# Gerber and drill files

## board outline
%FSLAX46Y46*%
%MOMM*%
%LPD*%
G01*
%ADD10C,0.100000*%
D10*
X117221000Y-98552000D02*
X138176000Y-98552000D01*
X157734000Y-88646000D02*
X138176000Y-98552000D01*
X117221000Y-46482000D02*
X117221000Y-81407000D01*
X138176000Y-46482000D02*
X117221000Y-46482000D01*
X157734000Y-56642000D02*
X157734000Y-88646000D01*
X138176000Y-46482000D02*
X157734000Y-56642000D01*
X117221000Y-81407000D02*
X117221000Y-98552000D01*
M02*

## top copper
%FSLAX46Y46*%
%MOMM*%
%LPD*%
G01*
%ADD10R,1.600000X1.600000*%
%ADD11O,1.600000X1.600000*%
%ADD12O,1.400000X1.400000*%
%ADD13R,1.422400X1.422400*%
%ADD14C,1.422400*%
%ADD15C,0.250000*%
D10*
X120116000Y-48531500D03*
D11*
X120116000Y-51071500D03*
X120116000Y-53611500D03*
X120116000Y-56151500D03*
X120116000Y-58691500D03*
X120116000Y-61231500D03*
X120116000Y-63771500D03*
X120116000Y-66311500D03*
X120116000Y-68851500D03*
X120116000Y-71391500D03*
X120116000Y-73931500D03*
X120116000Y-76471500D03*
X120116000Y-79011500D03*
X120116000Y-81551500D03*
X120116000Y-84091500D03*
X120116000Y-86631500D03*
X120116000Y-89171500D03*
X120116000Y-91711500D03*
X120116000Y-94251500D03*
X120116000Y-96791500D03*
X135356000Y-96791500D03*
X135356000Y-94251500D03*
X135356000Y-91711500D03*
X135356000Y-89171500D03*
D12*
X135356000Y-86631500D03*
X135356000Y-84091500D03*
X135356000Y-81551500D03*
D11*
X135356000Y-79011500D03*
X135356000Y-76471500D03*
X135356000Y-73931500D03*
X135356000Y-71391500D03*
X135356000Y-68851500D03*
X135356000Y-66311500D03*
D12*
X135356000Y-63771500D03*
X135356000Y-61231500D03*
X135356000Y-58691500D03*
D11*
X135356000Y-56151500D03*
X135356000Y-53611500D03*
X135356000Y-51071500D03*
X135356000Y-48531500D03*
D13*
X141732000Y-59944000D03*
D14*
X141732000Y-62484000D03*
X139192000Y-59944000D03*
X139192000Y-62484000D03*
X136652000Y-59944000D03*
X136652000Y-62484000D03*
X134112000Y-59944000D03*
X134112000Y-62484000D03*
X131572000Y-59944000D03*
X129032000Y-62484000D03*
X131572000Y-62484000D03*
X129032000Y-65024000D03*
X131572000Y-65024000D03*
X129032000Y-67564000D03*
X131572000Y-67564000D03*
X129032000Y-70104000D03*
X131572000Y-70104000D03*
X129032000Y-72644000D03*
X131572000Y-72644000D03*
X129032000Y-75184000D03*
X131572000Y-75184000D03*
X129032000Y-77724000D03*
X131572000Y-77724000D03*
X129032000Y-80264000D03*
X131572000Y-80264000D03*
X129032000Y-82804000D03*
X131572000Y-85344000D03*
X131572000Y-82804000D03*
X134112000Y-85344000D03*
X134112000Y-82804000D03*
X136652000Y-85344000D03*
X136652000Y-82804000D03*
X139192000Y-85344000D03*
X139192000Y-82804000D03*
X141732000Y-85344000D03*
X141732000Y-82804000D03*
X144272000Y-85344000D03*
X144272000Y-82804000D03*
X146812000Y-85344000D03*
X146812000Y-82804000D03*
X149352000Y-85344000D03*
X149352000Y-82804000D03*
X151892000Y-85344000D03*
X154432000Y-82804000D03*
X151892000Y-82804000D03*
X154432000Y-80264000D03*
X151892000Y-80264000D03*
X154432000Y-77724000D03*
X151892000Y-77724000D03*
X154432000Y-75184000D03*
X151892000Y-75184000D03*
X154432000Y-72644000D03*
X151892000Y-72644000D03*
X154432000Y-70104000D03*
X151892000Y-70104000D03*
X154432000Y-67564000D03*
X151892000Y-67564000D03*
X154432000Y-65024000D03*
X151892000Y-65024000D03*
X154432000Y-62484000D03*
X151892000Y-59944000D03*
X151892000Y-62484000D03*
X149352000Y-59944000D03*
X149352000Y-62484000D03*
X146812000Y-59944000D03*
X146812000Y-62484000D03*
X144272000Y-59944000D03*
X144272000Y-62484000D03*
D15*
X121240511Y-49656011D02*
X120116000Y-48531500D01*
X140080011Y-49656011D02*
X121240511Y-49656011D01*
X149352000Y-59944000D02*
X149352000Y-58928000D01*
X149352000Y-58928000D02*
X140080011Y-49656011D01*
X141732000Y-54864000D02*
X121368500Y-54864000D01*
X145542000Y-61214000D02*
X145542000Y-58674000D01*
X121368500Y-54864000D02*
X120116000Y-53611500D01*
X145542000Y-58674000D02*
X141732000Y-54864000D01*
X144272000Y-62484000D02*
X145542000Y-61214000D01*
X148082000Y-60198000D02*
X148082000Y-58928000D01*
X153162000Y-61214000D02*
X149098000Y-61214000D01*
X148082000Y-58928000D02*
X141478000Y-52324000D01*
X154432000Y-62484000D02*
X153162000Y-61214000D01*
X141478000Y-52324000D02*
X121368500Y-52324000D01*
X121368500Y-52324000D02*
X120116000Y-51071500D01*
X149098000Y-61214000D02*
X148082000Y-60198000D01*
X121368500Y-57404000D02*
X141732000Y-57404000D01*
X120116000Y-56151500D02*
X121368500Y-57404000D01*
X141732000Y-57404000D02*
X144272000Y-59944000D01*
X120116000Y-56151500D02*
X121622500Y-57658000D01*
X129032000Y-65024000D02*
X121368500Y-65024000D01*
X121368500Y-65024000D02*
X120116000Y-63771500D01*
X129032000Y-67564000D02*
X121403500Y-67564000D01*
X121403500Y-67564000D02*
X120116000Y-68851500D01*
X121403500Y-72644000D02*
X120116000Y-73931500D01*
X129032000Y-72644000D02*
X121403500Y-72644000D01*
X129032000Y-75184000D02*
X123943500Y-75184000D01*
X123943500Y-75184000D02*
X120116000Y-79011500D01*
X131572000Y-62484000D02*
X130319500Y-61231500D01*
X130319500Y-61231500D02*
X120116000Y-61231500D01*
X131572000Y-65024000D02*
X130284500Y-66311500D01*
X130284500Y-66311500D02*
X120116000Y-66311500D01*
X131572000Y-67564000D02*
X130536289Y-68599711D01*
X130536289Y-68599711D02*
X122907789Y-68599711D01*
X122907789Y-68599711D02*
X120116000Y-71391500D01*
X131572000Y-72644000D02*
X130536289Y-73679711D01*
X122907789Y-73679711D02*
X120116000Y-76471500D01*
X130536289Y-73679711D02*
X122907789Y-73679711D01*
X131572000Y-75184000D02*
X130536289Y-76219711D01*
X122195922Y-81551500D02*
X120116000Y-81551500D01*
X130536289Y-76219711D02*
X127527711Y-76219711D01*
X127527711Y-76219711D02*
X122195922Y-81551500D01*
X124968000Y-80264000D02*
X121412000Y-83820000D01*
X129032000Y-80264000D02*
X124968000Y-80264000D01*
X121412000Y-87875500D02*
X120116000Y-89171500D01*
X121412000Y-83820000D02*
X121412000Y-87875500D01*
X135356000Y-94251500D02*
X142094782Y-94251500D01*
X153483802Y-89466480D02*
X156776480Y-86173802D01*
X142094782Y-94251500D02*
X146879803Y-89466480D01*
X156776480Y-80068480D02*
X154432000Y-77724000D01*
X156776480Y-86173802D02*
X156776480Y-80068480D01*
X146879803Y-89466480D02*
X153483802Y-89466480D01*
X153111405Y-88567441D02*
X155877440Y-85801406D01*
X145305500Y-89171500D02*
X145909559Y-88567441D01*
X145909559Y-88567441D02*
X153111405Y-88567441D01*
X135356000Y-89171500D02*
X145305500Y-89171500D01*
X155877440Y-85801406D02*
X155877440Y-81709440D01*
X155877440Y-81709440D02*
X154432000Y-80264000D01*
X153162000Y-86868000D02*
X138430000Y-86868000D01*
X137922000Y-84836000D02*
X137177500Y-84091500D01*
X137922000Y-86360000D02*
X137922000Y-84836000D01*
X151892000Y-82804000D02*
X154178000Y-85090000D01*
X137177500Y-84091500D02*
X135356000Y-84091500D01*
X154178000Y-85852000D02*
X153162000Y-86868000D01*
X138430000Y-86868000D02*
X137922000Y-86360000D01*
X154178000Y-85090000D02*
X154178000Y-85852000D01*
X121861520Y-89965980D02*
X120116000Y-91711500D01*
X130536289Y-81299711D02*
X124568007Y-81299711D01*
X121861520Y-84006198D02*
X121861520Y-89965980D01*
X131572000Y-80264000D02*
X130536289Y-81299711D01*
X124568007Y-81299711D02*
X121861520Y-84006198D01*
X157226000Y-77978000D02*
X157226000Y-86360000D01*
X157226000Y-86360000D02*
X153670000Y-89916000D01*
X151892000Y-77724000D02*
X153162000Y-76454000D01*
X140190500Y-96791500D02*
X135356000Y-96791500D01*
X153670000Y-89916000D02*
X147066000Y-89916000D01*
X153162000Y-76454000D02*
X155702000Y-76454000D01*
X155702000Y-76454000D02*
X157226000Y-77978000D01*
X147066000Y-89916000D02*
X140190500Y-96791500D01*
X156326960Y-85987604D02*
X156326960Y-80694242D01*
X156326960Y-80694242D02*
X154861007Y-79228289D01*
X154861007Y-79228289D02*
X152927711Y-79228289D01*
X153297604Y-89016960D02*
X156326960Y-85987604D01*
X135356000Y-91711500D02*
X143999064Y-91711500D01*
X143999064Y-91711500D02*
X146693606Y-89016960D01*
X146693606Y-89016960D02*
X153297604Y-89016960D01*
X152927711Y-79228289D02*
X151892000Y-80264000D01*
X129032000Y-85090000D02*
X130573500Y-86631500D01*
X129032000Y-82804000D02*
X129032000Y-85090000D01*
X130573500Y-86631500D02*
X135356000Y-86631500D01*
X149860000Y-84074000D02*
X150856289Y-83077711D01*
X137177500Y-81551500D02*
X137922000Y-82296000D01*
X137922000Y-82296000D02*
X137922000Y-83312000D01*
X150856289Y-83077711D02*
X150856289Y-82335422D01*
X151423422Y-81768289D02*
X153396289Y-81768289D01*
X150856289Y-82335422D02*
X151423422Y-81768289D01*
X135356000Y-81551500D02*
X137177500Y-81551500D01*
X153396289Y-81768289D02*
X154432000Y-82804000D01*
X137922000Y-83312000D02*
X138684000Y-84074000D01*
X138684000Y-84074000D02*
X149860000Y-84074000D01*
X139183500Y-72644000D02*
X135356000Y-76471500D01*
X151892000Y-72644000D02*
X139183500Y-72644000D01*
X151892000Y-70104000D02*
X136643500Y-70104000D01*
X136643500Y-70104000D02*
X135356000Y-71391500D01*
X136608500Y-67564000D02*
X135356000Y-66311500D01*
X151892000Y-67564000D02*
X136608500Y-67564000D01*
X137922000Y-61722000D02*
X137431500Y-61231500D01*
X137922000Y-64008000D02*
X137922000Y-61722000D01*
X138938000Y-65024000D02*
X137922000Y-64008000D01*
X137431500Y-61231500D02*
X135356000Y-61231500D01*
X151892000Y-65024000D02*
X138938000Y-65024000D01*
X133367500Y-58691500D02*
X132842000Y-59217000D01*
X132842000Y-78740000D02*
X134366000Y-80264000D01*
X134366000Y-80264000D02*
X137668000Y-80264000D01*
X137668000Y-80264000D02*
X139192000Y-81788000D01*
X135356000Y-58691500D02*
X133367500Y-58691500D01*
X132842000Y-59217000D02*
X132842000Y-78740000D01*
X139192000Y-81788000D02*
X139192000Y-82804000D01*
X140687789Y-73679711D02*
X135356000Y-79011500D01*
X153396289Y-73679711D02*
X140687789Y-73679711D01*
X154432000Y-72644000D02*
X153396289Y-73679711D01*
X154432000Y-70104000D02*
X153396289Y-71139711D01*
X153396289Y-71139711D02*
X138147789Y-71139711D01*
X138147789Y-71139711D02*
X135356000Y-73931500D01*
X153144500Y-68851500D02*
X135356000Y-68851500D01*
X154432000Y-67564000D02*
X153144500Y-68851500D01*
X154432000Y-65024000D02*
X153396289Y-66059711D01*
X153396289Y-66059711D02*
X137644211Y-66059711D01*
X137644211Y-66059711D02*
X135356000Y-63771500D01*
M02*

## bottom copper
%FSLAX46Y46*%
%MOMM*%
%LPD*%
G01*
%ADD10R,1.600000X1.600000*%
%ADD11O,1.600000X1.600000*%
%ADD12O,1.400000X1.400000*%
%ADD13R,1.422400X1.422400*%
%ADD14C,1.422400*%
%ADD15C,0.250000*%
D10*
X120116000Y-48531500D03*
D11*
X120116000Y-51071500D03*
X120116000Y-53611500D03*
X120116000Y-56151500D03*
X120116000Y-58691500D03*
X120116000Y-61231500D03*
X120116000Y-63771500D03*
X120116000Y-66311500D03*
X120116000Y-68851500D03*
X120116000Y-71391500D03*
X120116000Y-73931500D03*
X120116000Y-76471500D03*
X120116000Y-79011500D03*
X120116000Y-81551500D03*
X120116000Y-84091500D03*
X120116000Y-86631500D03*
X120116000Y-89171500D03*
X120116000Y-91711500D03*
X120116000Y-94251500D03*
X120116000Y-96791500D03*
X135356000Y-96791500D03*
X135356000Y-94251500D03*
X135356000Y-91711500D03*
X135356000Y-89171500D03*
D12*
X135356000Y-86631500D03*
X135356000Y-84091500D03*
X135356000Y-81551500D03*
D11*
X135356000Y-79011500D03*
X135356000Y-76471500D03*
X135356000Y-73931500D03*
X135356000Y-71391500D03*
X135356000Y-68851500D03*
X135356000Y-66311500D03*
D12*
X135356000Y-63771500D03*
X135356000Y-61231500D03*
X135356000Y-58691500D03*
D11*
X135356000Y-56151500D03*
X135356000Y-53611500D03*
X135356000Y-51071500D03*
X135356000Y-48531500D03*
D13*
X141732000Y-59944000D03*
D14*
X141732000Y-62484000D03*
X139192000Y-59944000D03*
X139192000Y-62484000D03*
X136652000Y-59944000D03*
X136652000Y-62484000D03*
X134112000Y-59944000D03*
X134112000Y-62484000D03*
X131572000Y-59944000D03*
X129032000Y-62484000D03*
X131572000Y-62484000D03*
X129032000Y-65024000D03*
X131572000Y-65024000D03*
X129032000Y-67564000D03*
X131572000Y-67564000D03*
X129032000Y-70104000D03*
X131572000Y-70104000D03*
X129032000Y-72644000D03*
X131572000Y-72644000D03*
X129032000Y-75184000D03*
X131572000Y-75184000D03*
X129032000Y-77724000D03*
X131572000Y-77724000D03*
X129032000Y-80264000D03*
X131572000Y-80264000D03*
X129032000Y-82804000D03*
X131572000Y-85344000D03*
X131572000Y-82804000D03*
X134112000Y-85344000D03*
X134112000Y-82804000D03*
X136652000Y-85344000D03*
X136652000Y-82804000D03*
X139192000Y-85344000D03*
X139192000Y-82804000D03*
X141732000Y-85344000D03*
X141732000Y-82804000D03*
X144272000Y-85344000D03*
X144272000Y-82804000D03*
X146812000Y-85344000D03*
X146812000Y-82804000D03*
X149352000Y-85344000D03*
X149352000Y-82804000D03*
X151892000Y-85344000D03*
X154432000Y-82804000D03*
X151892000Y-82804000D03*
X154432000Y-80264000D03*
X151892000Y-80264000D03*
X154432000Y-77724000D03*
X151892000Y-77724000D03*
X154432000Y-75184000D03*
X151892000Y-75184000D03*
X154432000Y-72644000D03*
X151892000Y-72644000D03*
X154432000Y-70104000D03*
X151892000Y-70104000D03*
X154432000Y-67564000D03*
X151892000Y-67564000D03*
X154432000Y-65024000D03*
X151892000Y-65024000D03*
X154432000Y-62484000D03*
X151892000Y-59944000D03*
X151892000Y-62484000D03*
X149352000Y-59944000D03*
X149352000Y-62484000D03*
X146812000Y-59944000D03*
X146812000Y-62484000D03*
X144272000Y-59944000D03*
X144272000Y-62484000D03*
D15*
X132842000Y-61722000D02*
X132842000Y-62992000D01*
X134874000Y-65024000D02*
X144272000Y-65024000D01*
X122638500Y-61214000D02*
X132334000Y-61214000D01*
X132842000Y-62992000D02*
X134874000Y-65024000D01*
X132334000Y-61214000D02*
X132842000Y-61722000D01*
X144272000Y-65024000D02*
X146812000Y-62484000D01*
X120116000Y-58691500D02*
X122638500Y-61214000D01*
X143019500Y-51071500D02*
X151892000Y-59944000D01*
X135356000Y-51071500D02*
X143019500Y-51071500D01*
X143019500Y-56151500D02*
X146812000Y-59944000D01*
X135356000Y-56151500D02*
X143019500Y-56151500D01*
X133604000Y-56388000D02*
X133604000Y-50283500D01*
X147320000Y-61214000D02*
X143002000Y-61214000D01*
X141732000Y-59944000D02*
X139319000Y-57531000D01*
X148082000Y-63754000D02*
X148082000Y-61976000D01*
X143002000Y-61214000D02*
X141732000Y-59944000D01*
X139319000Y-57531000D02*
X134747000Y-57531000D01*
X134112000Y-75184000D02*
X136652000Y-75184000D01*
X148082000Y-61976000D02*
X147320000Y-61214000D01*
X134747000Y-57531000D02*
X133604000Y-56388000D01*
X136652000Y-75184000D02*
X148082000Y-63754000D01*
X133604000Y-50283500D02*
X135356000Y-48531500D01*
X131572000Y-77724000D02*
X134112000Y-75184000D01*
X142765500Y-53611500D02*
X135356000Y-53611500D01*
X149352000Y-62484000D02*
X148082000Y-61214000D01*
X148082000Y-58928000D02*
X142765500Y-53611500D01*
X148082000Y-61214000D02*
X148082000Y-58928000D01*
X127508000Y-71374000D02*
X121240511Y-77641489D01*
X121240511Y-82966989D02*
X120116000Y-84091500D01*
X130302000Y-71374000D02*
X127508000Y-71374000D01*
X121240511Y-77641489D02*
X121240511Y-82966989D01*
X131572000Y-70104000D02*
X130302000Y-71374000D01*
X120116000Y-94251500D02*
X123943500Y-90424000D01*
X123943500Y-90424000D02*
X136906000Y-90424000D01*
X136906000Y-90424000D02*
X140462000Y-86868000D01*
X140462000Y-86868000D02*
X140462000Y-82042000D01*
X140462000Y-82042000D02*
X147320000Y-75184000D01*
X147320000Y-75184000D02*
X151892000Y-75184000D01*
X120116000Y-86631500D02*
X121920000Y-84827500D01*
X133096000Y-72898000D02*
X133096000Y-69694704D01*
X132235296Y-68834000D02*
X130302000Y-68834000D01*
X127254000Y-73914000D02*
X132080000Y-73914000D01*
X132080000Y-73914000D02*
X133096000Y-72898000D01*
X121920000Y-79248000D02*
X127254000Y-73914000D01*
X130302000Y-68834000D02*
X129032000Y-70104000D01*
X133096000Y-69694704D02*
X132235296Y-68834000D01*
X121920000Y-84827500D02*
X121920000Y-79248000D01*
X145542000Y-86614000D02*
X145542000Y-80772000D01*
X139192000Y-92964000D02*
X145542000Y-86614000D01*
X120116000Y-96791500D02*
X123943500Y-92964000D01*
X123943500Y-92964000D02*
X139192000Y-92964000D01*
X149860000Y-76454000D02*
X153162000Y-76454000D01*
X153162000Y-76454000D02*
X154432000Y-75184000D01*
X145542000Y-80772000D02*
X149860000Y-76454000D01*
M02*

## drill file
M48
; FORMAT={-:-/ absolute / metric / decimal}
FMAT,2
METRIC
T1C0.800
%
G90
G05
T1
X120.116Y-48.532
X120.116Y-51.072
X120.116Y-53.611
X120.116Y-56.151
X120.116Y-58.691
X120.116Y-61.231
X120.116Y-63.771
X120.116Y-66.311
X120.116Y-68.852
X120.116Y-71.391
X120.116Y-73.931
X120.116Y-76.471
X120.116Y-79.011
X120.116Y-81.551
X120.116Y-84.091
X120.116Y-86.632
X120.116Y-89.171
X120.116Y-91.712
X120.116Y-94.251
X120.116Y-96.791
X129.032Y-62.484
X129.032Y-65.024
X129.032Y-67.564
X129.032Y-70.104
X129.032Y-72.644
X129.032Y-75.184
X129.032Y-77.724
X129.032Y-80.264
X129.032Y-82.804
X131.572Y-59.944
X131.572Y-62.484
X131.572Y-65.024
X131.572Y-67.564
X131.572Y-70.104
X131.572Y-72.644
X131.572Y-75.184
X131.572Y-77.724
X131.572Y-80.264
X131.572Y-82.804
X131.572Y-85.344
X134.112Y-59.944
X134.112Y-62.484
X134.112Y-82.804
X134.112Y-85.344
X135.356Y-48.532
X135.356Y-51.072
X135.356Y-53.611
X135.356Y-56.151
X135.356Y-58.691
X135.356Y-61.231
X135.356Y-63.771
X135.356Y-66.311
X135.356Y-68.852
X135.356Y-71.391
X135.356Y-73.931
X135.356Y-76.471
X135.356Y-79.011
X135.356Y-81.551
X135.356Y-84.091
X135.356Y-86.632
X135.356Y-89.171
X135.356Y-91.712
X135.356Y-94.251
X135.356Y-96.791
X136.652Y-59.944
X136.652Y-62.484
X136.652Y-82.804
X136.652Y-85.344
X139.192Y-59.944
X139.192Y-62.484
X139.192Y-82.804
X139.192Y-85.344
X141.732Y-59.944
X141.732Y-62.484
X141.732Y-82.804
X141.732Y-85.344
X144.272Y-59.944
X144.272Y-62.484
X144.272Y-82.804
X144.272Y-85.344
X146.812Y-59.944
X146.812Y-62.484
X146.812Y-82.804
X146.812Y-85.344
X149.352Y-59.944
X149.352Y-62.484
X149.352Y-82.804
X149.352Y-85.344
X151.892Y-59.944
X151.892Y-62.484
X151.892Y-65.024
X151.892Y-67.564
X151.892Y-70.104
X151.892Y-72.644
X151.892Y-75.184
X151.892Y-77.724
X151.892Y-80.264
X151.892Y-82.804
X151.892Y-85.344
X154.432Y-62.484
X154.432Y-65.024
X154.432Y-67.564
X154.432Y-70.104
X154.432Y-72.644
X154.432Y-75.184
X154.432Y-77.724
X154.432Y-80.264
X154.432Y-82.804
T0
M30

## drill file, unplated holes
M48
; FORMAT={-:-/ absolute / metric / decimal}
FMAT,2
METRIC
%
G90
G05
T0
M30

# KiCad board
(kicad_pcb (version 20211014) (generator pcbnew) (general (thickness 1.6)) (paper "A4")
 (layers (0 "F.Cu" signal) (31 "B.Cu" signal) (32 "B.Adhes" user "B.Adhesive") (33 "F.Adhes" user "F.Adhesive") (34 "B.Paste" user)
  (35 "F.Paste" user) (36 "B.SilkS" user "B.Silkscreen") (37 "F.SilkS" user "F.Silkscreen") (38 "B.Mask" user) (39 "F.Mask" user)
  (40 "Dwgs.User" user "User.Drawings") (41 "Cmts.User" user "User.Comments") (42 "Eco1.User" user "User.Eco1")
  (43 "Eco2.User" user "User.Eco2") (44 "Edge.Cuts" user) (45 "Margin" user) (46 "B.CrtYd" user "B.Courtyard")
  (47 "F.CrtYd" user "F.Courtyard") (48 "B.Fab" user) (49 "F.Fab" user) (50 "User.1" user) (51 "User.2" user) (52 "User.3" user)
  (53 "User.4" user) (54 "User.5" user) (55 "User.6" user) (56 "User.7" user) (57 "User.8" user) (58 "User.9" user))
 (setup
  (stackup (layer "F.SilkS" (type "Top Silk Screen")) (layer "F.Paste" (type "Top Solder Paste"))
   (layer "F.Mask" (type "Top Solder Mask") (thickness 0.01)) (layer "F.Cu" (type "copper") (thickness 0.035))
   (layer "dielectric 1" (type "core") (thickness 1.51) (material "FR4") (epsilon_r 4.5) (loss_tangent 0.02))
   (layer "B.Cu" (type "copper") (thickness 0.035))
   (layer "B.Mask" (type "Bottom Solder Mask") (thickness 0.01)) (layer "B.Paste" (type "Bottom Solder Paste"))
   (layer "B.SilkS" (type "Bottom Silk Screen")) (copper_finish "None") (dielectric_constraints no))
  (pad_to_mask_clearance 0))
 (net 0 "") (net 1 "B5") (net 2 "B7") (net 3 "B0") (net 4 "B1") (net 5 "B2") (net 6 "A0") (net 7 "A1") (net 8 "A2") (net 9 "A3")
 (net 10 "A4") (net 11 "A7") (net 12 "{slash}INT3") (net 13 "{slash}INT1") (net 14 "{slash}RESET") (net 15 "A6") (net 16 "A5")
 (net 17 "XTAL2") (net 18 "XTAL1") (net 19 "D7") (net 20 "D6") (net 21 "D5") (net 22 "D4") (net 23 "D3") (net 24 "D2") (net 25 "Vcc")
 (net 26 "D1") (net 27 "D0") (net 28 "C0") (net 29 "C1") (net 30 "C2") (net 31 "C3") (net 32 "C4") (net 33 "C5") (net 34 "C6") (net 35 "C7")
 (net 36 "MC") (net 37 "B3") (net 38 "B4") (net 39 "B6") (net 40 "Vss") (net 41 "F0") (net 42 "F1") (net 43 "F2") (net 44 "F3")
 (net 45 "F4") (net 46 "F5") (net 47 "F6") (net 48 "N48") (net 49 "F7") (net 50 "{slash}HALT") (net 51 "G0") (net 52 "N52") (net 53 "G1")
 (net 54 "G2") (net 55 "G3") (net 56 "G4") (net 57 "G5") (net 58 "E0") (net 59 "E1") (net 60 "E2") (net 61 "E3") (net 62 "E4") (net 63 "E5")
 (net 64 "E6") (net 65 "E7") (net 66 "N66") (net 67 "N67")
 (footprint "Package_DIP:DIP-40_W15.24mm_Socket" (layer "F.Cu") (at 120.116 48.5315)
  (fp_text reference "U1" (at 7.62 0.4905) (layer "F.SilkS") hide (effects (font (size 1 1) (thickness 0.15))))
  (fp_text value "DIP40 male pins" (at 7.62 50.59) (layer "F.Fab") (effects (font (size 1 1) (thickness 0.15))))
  (pad "1" thru_hole rect locked (at 0 0) (size 1.6 1.6) (drill 0.8) (layers *.Cu *.Mask) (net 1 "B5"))
  (pad "2" thru_hole oval locked (at 0 2.54) (size 1.6 1.6) (drill 0.8) (layers *.Cu *.Mask) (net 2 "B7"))
  (pad "3" thru_hole oval locked (at 0 5.08) (size 1.6 1.6) (drill 0.8) (layers *.Cu *.Mask) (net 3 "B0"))
  (pad "4" thru_hole oval locked (at 0 7.62) (size 1.6 1.6) (drill 0.8) (layers *.Cu *.Mask) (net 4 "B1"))
  (pad "5" thru_hole oval locked (at 0 10.16) (size 1.6 1.6) (drill 0.8) (layers *.Cu *.Mask) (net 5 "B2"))
  (pad "6" thru_hole oval locked (at 0 12.7) (size 1.6 1.6) (drill 0.8) (layers *.Cu *.Mask) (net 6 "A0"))
  (pad "7" thru_hole oval locked (at 0 15.24) (size 1.6 1.6) (drill 0.8) (layers *.Cu *.Mask) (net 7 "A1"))
  (pad "8" thru_hole oval locked (at 0 17.78) (size 1.6 1.6) (drill 0.8) (layers *.Cu *.Mask) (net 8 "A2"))
  (pad "9" thru_hole oval locked (at 0 20.32) (size 1.6 1.6) (drill 0.8) (layers *.Cu *.Mask) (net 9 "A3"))
  (pad "10" thru_hole oval locked (at 0 22.86) (size 1.6 1.6) (drill 0.8) (layers *.Cu *.Mask) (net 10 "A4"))
  (pad "11" thru_hole oval locked (at 0 25.4) (size 1.6 1.6) (drill 0.8) (layers *.Cu *.Mask) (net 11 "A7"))
  (pad "12" thru_hole oval locked (at 0 27.94) (size 1.6 1.6) (drill 0.8) (layers *.Cu *.Mask) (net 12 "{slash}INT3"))
  (pad "13" thru_hole oval locked (at 0 30.48) (size 1.6 1.6) (drill 0.8) (layers *.Cu *.Mask) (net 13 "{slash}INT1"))
  (pad "14" thru_hole oval locked (at 0 33.02) (size 1.6 1.6) (drill 0.8) (layers *.Cu *.Mask) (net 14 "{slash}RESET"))
  (pad "15" thru_hole oval locked (at 0 35.56) (size 1.6 1.6) (drill 0.8) (layers *.Cu *.Mask) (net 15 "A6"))
  (pad "16" thru_hole oval locked (at 0 38.1) (size 1.6 1.6) (drill 0.8) (layers *.Cu *.Mask) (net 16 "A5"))
  (pad "17" thru_hole oval locked (at 0 40.64) (size 1.6 1.6) (drill 0.8) (layers *.Cu *.Mask) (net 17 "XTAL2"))
  (pad "18" thru_hole oval locked (at 0 43.18) (size 1.6 1.6) (drill 0.8) (layers *.Cu *.Mask) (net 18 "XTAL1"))
  (pad "19" thru_hole oval locked (at 0 45.72) (size 1.6 1.6) (drill 0.8) (layers *.Cu *.Mask) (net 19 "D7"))
  (pad "20" thru_hole oval locked (at 0 48.26) (size 1.6 1.6) (drill 0.8) (layers *.Cu *.Mask) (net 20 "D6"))
  (pad "21" thru_hole oval locked (at 15.24 48.26) (size 1.6 1.6) (drill 0.8) (layers *.Cu *.Mask) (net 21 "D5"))
  (pad "22" thru_hole oval locked (at 15.24 45.72) (size 1.6 1.6) (drill 0.8) (layers *.Cu *.Mask) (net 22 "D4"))
  (pad "23" thru_hole oval locked (at 15.24 43.18) (size 1.6 1.6) (drill 0.8) (layers *.Cu *.Mask) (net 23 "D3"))
  (pad "24" thru_hole oval locked (at 15.24 40.64) (size 1.6 1.6) (drill 0.8) (layers *.Cu *.Mask) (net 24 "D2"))
  (pad "25" thru_hole oval locked (at 15.24 38.1) (size 1.4 1.4) (drill 0.8) (layers *.Cu *.Mask) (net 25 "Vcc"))
  (pad "26" thru_hole oval locked (at 15.24 35.56) (size 1.4 1.4) (drill 0.8) (layers *.Cu *.Mask) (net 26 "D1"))
  (pad "27" thru_hole oval locked (at 15.24 33.02) (size 1.4 1.4) (drill 0.8) (layers *.Cu *.Mask) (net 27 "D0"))
  (pad "28" thru_hole oval locked (at 15.24 30.48) (size 1.6 1.6) (drill 0.8) (layers *.Cu *.Mask) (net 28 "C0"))
  (pad "29" thru_hole oval locked (at 15.24 27.94) (size 1.6 1.6) (drill 0.8) (layers *.Cu *.Mask) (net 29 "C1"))
  (pad "30" thru_hole oval locked (at 15.24 25.4) (size 1.6 1.6) (drill 0.8) (layers *.Cu *.Mask) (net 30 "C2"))
  (pad "31" thru_hole oval locked (at 15.24 22.86) (size 1.6 1.6) (drill 0.8) (layers *.Cu *.Mask) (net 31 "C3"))
  (pad "32" thru_hole oval locked (at 15.24 20.32) (size 1.6 1.6) (drill 0.8) (layers *.Cu *.Mask) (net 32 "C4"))
  (pad "33" thru_hole oval locked (at 15.24 17.78) (size 1.6 1.6) (drill 0.8) (layers *.Cu *.Mask) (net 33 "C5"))
  (pad "34" thru_hole oval locked (at 15.24 15.24) (size 1.4 1.4) (drill 0.8) (layers *.Cu *.Mask) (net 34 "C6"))
  (pad "35" thru_hole oval locked (at 15.24 12.7) (size 1.4 1.4) (drill 0.8) (layers *.Cu *.Mask) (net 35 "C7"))
  (pad "36" thru_hole oval locked (at 15.24 10.16) (size 1.4 1.4) (drill 0.8) (layers *.Cu *.Mask) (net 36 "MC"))
  (pad "37" thru_hole oval locked (at 15.24 7.62) (size 1.6 1.6) (drill 0.8) (layers *.Cu *.Mask) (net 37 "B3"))
  (pad "38" thru_hole oval locked (at 15.24 5.08) (size 1.6 1.6) (drill 0.8) (layers *.Cu *.Mask) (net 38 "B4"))
  (pad "39" thru_hole oval locked (at 15.24 2.54) (size 1.6 1.6) (drill 0.8) (layers *.Cu *.Mask) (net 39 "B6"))
  (pad "40" thru_hole oval locked (at 15.24 0) (size 1.6 1.6) (drill 0.8) (layers *.Cu *.Mask) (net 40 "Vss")))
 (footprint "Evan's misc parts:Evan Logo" (layer "F.Cu") (at 127.381 91.567)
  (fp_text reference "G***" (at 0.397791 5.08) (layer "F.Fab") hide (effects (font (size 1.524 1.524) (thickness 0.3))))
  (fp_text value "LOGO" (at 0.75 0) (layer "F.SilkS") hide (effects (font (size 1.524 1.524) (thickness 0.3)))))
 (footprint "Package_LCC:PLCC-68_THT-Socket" (layer "F.Cu") (at 141.732 59.944)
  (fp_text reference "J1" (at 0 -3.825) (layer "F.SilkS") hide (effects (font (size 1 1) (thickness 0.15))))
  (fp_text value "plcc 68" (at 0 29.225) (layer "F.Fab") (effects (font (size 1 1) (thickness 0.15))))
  (pad "1" thru_hole rect locked (at 0 0) (size 1.4224 1.4224) (drill 0.8) (layers *.Cu *.Mask) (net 40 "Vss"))
  (pad "2" thru_hole circle locked (at 0 2.54) (size 1.4224 1.4224) (drill 0.8) (layers *.Cu *.Mask) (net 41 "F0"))
  (pad "3" thru_hole circle locked (at -2.54 0) (size 1.4224 1.4224) (drill 0.8) (layers *.Cu *.Mask) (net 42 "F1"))
  (pad "4" thru_hole circle locked (at -2.54 2.54) (size 1.4224 1.4224) (drill 0.8) (layers *.Cu *.Mask) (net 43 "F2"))
  (pad "5" thru_hole circle locked (at -5.08 0) (size 1.4224 1.4224) (drill 0.8) (layers *.Cu *.Mask) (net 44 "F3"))
  (pad "6" thru_hole circle locked (at -5.08 2.54) (size 1.4224 1.4224) (drill 0.8) (layers *.Cu *.Mask) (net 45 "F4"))
  (pad "7" thru_hole circle locked (at -7.62 0) (size 1.4224 1.4224) (drill 0.8) (layers *.Cu *.Mask) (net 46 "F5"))
  (pad "8" thru_hole circle locked (at -7.62 2.54) (size 1.4224 1.4224) (drill 0.8) (layers *.Cu *.Mask) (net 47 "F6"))
  (pad "9" thru_hole circle locked (at -10.16 0) (size 1.4224 1.4224) (drill 0.8) (layers *.Cu *.Mask) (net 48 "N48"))
  (pad "10" thru_hole circle locked (at -12.7 2.54) (size 1.4224 1.4224) (drill 0.8) (layers *.Cu *.Mask) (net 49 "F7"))
  (pad "11" thru_hole circle locked (at -10.16 2.54) (size 1.4224 1.4224) (drill 0.8) (layers *.Cu *.Mask) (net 6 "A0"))
  (pad "12" thru_hole circle locked (at -12.7 5.08) (size 1.4224 1.4224) (drill 0.8) (layers *.Cu *.Mask) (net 7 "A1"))
  (pad "13" thru_hole circle locked (at -10.16 5.08) (size 1.4224 1.4224) (drill 0.8) (layers *.Cu *.Mask) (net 8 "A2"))
  (pad "14" thru_hole circle locked (at -12.7 7.62) (size 1.4224 1.4224) (drill 0.8) (layers *.Cu *.Mask) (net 9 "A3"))
  (pad "15" thru_hole circle locked (at -10.16 7.62) (size 1.4224 1.4224) (drill 0.8) (layers *.Cu *.Mask) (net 10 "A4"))
  (pad "16" thru_hole circle locked (at -12.7 10.16) (size 1.4224 1.4224) (drill 0.8) (layers *.Cu *.Mask) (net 16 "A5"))
  (pad "17" thru_hole circle locked (at -10.16 10.16) (size 1.4224 1.4224) (drill 0.8) (layers *.Cu *.Mask) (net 15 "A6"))
  (pad "18" thru_hole circle locked (at -12.7 12.7) (size 1.4224 1.4224) (drill 0.8) (layers *.Cu *.Mask) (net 11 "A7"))
  (pad "19" thru_hole circle locked (at -10.16 12.7) (size 1.4224 1.4224) (drill 0.8) (layers *.Cu *.Mask) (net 12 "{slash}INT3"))
  (pad "20" thru_hole circle locked (at -12.7 15.24) (size 1.4224 1.4224) (drill 0.8) (layers *.Cu *.Mask) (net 13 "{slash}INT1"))
  (pad "21" thru_hole circle locked (at -10.16 15.24) (size 1.4224 1.4224) (drill 0.8) (layers *.Cu *.Mask) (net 14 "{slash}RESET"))
  (pad "22" thru_hole circle locked (at -12.7 17.78) (size 1.4224 1.4224) (drill 0.8) (layers *.Cu *.Mask) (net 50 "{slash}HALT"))
  (pad "23" thru_hole circle locked (at -10.16 17.78) (size 1.4224 1.4224) (drill 0.8) (layers *.Cu *.Mask) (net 40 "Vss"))
  (pad "24" thru_hole circle locked (at -12.7 20.32) (size 1.4224 1.4224) (drill 0.8) (layers *.Cu *.Mask) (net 17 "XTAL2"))
  (pad "25" thru_hole circle locked (at -10.16 20.32) (size 1.4224 1.4224) (drill 0.8) (layers *.Cu *.Mask) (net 18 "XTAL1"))
  (pad "26" thru_hole circle locked (at -12.7 22.86) (size 1.4224 1.4224) (drill 0.8) (layers *.Cu *.Mask) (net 25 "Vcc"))
  (pad "27" thru_hole circle locked (at -10.16 25.4) (size 1.4224 1.4224) (drill 0.8) (layers *.Cu *.Mask) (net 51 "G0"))
  (pad "28" thru_hole circle locked (at -10.16 22.86) (size 1.4224 1.4224) (drill 0.8) (layers *.Cu *.Mask) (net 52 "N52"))
  (pad "29" thru_hole circle locked (at -7.62 25.4) (size 1.4224 1.4224) (drill 0.8) (layers *.Cu *.Mask) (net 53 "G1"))
  (pad "30" thru_hole circle locked (at -7.62 22.86) (size 1.4224 1.4224) (drill 0.8) (layers *.Cu *.Mask) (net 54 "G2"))
  (pad "31" thru_hole circle locked (at -5.08 25.4) (size 1.4224 1.4224) (drill 0.8) (layers *.Cu *.Mask) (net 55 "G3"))
  (pad "32" thru_hole circle locked (at -5.08 22.86) (size 1.4224 1.4224) (drill 0.8) (layers *.Cu *.Mask) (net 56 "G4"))
  (pad "33" thru_hole circle locked (at -2.54 25.4) (size 1.4224 1.4224) (drill 0.8) (layers *.Cu *.Mask) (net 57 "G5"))
  (pad "34" thru_hole circle locked (at -2.54 22.86) (size 1.4224 1.4224) (drill 0.8) (layers *.Cu *.Mask) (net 36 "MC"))
  (pad "35" thru_hole circle locked (at 0 25.4) (size 1.4224 1.4224) (drill 0.8) (layers *.Cu *.Mask) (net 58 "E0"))
  (pad "36" thru_hole circle locked (at 0 22.86) (size 1.4224 1.4224) (drill 0.8) (layers *.Cu *.Mask) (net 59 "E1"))
  (pad "37" thru_hole circle locked (at 2.54 25.4) (size 1.4224 1.4224) (drill 0.8) (layers *.Cu *.Mask) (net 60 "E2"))
  (pad "38" thru_hole circle locked (at 2.54 22.86) (size 1.4224 1.4224) (drill 0.8) (layers *.Cu *.Mask) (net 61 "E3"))
  (pad "39" thru_hole circle locked (at 5.08 25.4) (size 1.4224 1.4224) (drill 0.8) (layers *.Cu *.Mask) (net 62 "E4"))
  (pad "40" thru_hole circle locked (at 5.08 22.86) (size 1.4224 1.4224) (drill 0.8) (layers *.Cu *.Mask) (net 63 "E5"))
  (pad "41" thru_hole circle locked (at 7.62 25.4) (size 1.4224 1.4224) (drill 0.8) (layers *.Cu *.Mask) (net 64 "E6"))
  (pad "42" thru_hole circle locked (at 7.62 22.86) (size 1.4224 1.4224) (drill 0.8) (layers *.Cu *.Mask) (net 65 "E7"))
  (pad "43" thru_hole circle locked (at 10.16 25.4) (size 1.4224 1.4224) (drill 0.8) (layers *.Cu *.Mask) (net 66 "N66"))
  (pad "44" thru_hole circle locked (at 12.7 22.86) (size 1.4224 1.4224) (drill 0.8) (layers *.Cu *.Mask) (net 27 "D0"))
  (pad "45" thru_hole circle locked (at 10.16 22.86) (size 1.4224 1.4224) (drill 0.8) (layers *.Cu *.Mask) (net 26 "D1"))
  (pad "46" thru_hole circle locked (at 12.7 20.32) (size 1.4224 1.4224) (drill 0.8) (layers *.Cu *.Mask) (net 24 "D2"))
  (pad "47" thru_hole circle locked (at 10.16 20.32) (size 1.4224 1.4224) (drill 0.8) (layers *.Cu *.Mask) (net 23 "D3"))
  (pad "48" thru_hole circle locked (at 12.7 17.78) (size 1.4224 1.4224) (drill 0.8) (layers *.Cu *.Mask) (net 22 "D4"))
  (pad "49" thru_hole circle locked (at 10.16 17.78) (size 1.4224 1.4224) (drill 0.8) (layers *.Cu *.Mask) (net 21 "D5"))
  (pad "50" thru_hole circle locked (at 12.7 15.24) (size 1.4224 1.4224) (drill 0.8) (layers *.Cu *.Mask) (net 20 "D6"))
  (pad "51" thru_hole circle locked (at 10.16 15.24) (size 1.4224 1.4224) (drill 0.8) (layers *.Cu *.Mask) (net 19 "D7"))
  (pad "52" thru_hole circle locked (at 12.7 12.7) (size 1.4224 1.4224) (drill 0.8) (layers *.Cu *.Mask) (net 28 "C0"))
  (pad "53" thru_hole circle locked (at 10.16 12.7) (size 1.4224 1.4224) (drill 0.8) (layers *.Cu *.Mask) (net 29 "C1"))
  (pad "54" thru_hole circle locked (at 12.7 10.16) (size 1.4224 1.4224) (drill 0.8) (layers *.Cu *.Mask) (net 30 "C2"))
  (pad "55" thru_hole circle locked (at 10.16 10.16) (size 1.4224 1.4224) (drill 0.8) (layers *.Cu *.Mask) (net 31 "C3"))
  (pad "56" thru_hole circle locked (at 12.7 7.62) (size 1.4224 1.4224) (drill 0.8) (layers *.Cu *.Mask) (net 32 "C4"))
  (pad "57" thru_hole circle locked (at 10.16 7.62) (size 1.4224 1.4224) (drill 0.8) (layers *.Cu *.Mask) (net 33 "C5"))
  (pad "58" thru_hole circle locked (at 12.7 5.08) (size 1.4224 1.4224) (drill 0.8) (layers *.Cu *.Mask) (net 34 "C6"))
  (pad "59" thru_hole circle locked (at 10.16 5.08) (size 1.4224 1.4224) (drill 0.8) (layers *.Cu *.Mask) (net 35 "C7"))
  (pad "60" thru_hole circle locked (at 12.7 2.54) (size 1.4224 1.4224) (drill 0.8) (layers *.Cu *.Mask) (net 2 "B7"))
  (pad "61" thru_hole circle locked (at 10.16 0) (size 1.4224 1.4224) (drill 0.8) (layers *.Cu *.Mask) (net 39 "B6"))
  (pad "62" thru_hole circle locked (at 10.16 2.54) (size 1.4224 1.4224) (drill 0.8) (layers *.Cu *.Mask) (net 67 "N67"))
  (pad "63" thru_hole circle locked (at 7.62 0) (size 1.4224 1.4224) (drill 0.8) (layers *.Cu *.Mask) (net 1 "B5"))
  (pad "64" thru_hole circle locked (at 7.62 2.54) (size 1.4224 1.4224) (drill 0.8) (layers *.Cu *.Mask) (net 38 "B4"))
  (pad "65" thru_hole circle locked (at 5.08 0) (size 1.4224 1.4224) (drill 0.8) (layers *.Cu *.Mask) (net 37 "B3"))
  (pad "66" thru_hole circle locked (at 5.08 2.54) (size 1.4224 1.4224) (drill 0.8) (layers *.Cu *.Mask) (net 5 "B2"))
  (pad "67" thru_hole circle locked (at 2.54 0) (size 1.4224 1.4224) (drill 0.8) (layers *.Cu *.Mask) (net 4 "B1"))
  (pad "68" thru_hole circle locked (at 2.54 2.54) (size 1.4224 1.4224) (drill 0.8) (layers *.Cu *.Mask) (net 3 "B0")))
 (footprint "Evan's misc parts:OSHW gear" (layer "B.Cu") (at 127.381 90.932 180)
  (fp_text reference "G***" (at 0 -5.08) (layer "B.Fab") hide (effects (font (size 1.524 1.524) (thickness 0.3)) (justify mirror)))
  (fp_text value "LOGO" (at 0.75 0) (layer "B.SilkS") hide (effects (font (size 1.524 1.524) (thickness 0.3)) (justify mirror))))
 (gr_line (start 117.221 98.552) (end 138.176 98.552) (layer "Edge.Cuts") (width 0.1))
 (gr_line (start 157.734 88.646) (end 138.176 98.552) (layer "Edge.Cuts") (width 0.1))
 (gr_line (start 117.221 46.482) (end 117.221 81.407) (layer "Edge.Cuts") (width 0.1))
 (gr_line (start 138.176 46.482) (end 117.221 46.482) (layer "Edge.Cuts") (width 0.1))
 (gr_line (start 157.734 56.642) (end 157.734 88.646) (layer "Edge.Cuts") (width 0.1))
 (gr_line (start 138.176 46.482) (end 157.734 56.642) (layer "Edge.Cuts") (width 0.1))
 (gr_line (start 117.221 81.407) (end 117.221 98.552) (layer "Edge.Cuts") (width 0.1))
 (segment (start 121.240511 49.656011) (end 120.116 48.5315) (width 0.25) (layer "F.Cu") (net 1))
 (segment (start 140.080011 49.656011) (end 121.240511 49.656011) (width 0.25) (layer "F.Cu") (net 1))
 (segment (start 149.352 59.944) (end 149.352 58.928) (width 0.25) (layer "F.Cu") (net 1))
 (segment (start 149.352 58.928) (end 140.080011 49.656011) (width 0.25) (layer "F.Cu") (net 1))
 (segment (start 141.732 54.864) (end 121.3685 54.864) (width 0.25) (layer "F.Cu") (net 3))
 (segment (start 145.542 61.214) (end 145.542 58.674) (width 0.25) (layer "F.Cu") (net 3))
 (segment (start 121.3685 54.864) (end 120.116 53.6115) (width 0.25) (layer "F.Cu") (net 3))
 (segment (start 145.542 58.674) (end 141.732 54.864) (width 0.25) (layer "F.Cu") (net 3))
 (segment (start 144.272 62.484) (end 145.542 61.214) (width 0.25) (layer "F.Cu") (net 3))
 (segment (start 132.842 61.722) (end 132.842 62.992) (width 0.25) (layer "B.Cu") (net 5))
 (segment (start 134.874 65.024) (end 144.272 65.024) (width 0.25) (layer "B.Cu") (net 5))
 (segment (start 122.6385 61.214) (end 132.334 61.214) (width 0.25) (layer "B.Cu") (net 5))
 (segment (start 132.842 62.992) (end 134.874 65.024) (width 0.25) (layer "B.Cu") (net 5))
 (segment (start 132.334 61.214) (end 132.842 61.722) (width 0.25) (layer "B.Cu") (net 5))
 (segment (start 144.272 65.024) (end 146.812 62.484) (width 0.25) (layer "B.Cu") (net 5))
 (segment (start 120.116 58.6915) (end 122.6385 61.214) (width 0.25) (layer "B.Cu") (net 5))
 (segment (start 143.0195 51.0715) (end 151.892 59.944) (width 0.25) (layer "B.Cu") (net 39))
 (segment (start 135.356 51.0715) (end 143.0195 51.0715) (width 0.25) (layer "B.Cu") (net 39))
 (segment (start 143.0195 56.1515) (end 146.812 59.944) (width 0.25) (layer "B.Cu") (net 37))
 (segment (start 135.356 56.1515) (end 143.0195 56.1515) (width 0.25) (layer "B.Cu") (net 37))
 (segment (start 148.082 60.198) (end 148.082 58.928) (width 0.25) (layer "F.Cu") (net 2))
 (segment (start 153.162 61.214) (end 149.098 61.214) (width 0.25) (layer "F.Cu") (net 2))
 (segment (start 148.082 58.928) (end 141.478 52.324) (width 0.25) (layer "F.Cu") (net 2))
 (segment (start 154.432 62.484) (end 153.162 61.214) (width 0.25) (layer "F.Cu") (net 2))
 (segment (start 141.478 52.324) (end 121.3685 52.324) (width 0.25) (layer "F.Cu") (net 2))
 (segment (start 121.3685 52.324) (end 120.116 51.0715) (width 0.25) (layer "F.Cu") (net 2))
 (segment (start 149.098 61.214) (end 148.082 60.198) (width 0.25) (layer "F.Cu") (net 2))
 (segment (start 121.3685 57.404) (end 141.732 57.404) (width 0.25) (layer "F.Cu") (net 4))
 (segment (start 120.116 56.1515) (end 121.3685 57.404) (width 0.25) (layer "F.Cu") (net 4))
 (segment (start 141.732 57.404) (end 144.272 59.944) (width 0.25) (layer "F.Cu") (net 4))
 (segment (start 120.116 56.1515) (end 121.6225 57.658) (width 0.25) (layer "F.Cu") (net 4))
 (segment (start 133.604 56.388) (end 133.604 50.2835) (width 0.25) (layer "B.Cu") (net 40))
 (segment (start 147.32 61.214) (end 143.002 61.214) (width 0.25) (layer "B.Cu") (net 40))
 (segment (start 141.732 59.944) (end 139.319 57.531) (width 0.25) (layer "B.Cu") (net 40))
 (segment (start 148.082 63.754) (end 148.082 61.976) (width 0.25) (layer "B.Cu") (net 40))
 (segment (start 143.002 61.214) (end 141.732 59.944) (width 0.25) (layer "B.Cu") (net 40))
 (segment (start 139.319 57.531) (end 134.747 57.531) (width 0.25) (layer "B.Cu") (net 40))
 (segment (start 134.112 75.184) (end 136.652 75.184) (width 0.25) (layer "B.Cu") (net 40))
 (segment (start 148.082 61.976) (end 147.32 61.214) (width 0.25) (layer "B.Cu") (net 40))
 (segment (start 134.747 57.531) (end 133.604 56.388) (width 0.25) (layer "B.Cu") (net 40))
 (segment (start 136.652 75.184) (end 148.082 63.754) (width 0.25) (layer "B.Cu") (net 40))
 (segment (start 133.604 50.2835) (end 135.356 48.5315) (width 0.25) (layer "B.Cu") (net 40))
 (segment (start 131.572 77.724) (end 134.112 75.184) (width 0.25) (layer "B.Cu") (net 40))
 (segment (start 142.7655 53.6115) (end 135.356 53.6115) (width 0.25) (layer "B.Cu") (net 38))
 (segment (start 149.352 62.484) (end 148.082 61.214) (width 0.25) (layer "B.Cu") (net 38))
 (segment (start 148.082 58.928) (end 142.7655 53.6115) (width 0.25) (layer "B.Cu") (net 38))
 (segment (start 148.082 61.214) (end 148.082 58.928) (width 0.25) (layer "B.Cu") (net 38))
 (segment (start 129.032 65.024) (end 121.3685 65.024) (width 0.25) (layer "F.Cu") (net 7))
 (segment (start 121.3685 65.024) (end 120.116 63.7715) (width 0.25) (layer "F.Cu") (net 7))
 (segment (start 129.032 67.564) (end 121.4035 67.564) (width 0.25) (layer "F.Cu") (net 9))
 (segment (start 121.4035 67.564) (end 120.116 68.8515) (width 0.25) (layer "F.Cu") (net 9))
 (segment (start 121.4035 72.644) (end 120.116 73.9315) (width 0.25) (layer "F.Cu") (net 11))
 (segment (start 129.032 72.644) (end 121.4035 72.644) (width 0.25) (layer "F.Cu") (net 11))
 (segment (start 129.032 75.184) (end 123.9435 75.184) (width 0.25) (layer "F.Cu") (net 13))
 (segment (start 123.9435 75.184) (end 120.116 79.0115) (width 0.25) (layer "F.Cu") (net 13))
 (segment (start 127.508 71.374) (end 121.240511 77.641489) (width 0.25) (layer "B.Cu") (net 15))
 (segment (start 121.240511 82.966989) (end 120.116 84.0915) (width 0.25) (layer "B.Cu") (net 15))
 (segment (start 130.302 71.374) (end 127.508 71.374) (width 0.25) (layer "B.Cu") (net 15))
 (segment (start 121.240511 77.641489) (end 121.240511 82.966989) (width 0.25) (layer "B.Cu") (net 15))
 (segment (start 131.572 70.104) (end 130.302 71.374) (width 0.25) (layer "B.Cu") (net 15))
 (segment (start 131.572 62.484) (end 130.3195 61.2315) (width 0.25) (layer "F.Cu") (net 6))
 (segment (start 130.3195 61.2315) (end 120.116 61.2315) (width 0.25) (layer "F.Cu") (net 6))
 (segment (start 131.572 65.024) (end 130.2845 66.3115) (width 0.25) (layer "F.Cu") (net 8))
 (segment (start 130.2845 66.3115) (end 120.116 66.3115) (width 0.25) (layer "F.Cu") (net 8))
 (segment (start 131.572 67.564) (end 130.536289 68.599711) (width 0.25) (layer "F.Cu") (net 10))
 (segment (start 130.536289 68.599711) (end 122.907789 68.599711) (width 0.25) (layer "F.Cu") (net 10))
 (segment (start 122.907789 68.599711) (end 120.116 71.3915) (width 0.25) (layer "F.Cu") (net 10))
 (segment (start 131.572 72.644) (end 130.536289 73.679711) (width 0.25) (layer "F.Cu") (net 12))
 (segment (start 122.907789 73.679711) (end 120.116 76.4715) (width 0.25) (layer "F.Cu") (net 12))
 (segment (start 130.536289 73.679711) (end 122.907789 73.679711) (width 0.25) (layer "F.Cu") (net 12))
 (segment (start 131.572 75.184) (end 130.536289 76.219711) (width 0.25) (layer "F.Cu") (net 14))
 (segment (start 122.195922 81.5515) (end 120.116 81.5515) (width 0.25) (layer "F.Cu") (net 14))
 (segment (start 130.536289 76.219711) (end 127.527711 76.219711) (width 0.25) (layer "F.Cu") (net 14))
 (segment (start 127.527711 76.219711) (end 122.195922 81.5515) (width 0.25) (layer "F.Cu") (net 14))
 (segment (start 124.968 80.264) (end 121.412 83.82) (width 0.25) (layer "F.Cu") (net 17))
 (segment (start 129.032 80.264) (end 124.968 80.264) (width 0.25) (layer "F.Cu") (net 17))
 (segment (start 121.412 87.8755) (end 120.116 89.1715) (width 0.25) (layer "F.Cu") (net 17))
 (segment (start 121.412 83.82) (end 121.412 87.8755) (width 0.25) (layer "F.Cu") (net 17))
 (segment (start 120.116 94.2515) (end 123.9435 90.424) (width 0.25) (layer "B.Cu") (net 19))
 (segment (start 123.9435 90.424) (end 136.906 90.424) (width 0.25) (layer "B.Cu") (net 19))
 (segment (start 136.906 90.424) (end 140.462 86.868) (width 0.25) (layer "B.Cu") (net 19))
 (segment (start 140.462 86.868) (end 140.462 82.042) (width 0.25) (layer "B.Cu") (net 19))
 (segment (start 140.462 82.042) (end 147.32 75.184) (width 0.25) (layer "B.Cu") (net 19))
 (segment (start 147.32 75.184) (end 151.892 75.184) (width 0.25) (layer "B.Cu") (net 19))
 (segment (start 135.356 94.2515) (end 142.094782 94.2515) (width 0.25) (layer "F.Cu") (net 22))
 (segment (start 153.483802 89.46648) (end 156.77648 86.173802) (width 0.25) (layer "F.Cu") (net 22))
 (segment (start 142.094782 94.2515) (end 146.879803 89.46648) (width 0.25) (layer "F.Cu") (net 22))
 (segment (start 156.77648 80.06848) (end 154.432 77.724) (width 0.25) (layer "F.Cu") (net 22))
 (segment (start 156.77648 86.173802) (end 156.77648 80.06848) (width 0.25) (layer "F.Cu") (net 22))
 (segment (start 146.879803 89.46648) (end 153.483802 89.46648) (width 0.25) (layer "F.Cu") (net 22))
 (segment (start 153.111405 88.567441) (end 155.87744 85.801406) (width 0.25) (layer "F.Cu") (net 24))
 (segment (start 145.3055 89.1715) (end 145.909559 88.567441) (width 0.25) (layer "F.Cu") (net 24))
 (segment (start 145.909559 88.567441) (end 153.111405 88.567441) (width 0.25) (layer "F.Cu") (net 24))
 (segment (start 135.356 89.1715) (end 145.3055 89.1715) (width 0.25) (layer "F.Cu") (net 24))
 (segment (start 155.87744 85.801406) (end 155.87744 81.70944) (width 0.25) (layer "F.Cu") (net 24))
 (segment (start 155.87744 81.70944) (end 154.432 80.264) (width 0.25) (layer "F.Cu") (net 24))
 (segment (start 153.162 86.868) (end 138.43 86.868) (width 0.25) (layer "F.Cu") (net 26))
 (segment (start 137.922 84.836) (end 137.1775 84.0915) (width 0.25) (layer "F.Cu") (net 26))
 (segment (start 137.922 86.36) (end 137.922 84.836) (width 0.25) (layer "F.Cu") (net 26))
 (segment (start 151.892 82.804) (end 154.178 85.09) (width 0.25) (layer "F.Cu") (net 26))
 (segment (start 137.1775 84.0915) (end 135.356 84.0915) (width 0.25) (layer "F.Cu") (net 26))
 (segment (start 154.178 85.852) (end 153.162 86.868) (width 0.25) (layer "F.Cu") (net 26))
 (segment (start 138.43 86.868) (end 137.922 86.36) (width 0.25) (layer "F.Cu") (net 26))
 (segment (start 154.178 85.09) (end 154.178 85.852) (width 0.25) (layer "F.Cu") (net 26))
 (segment (start 120.116 86.6315) (end 121.92 84.8275) (width 0.25) (layer "B.Cu") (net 16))
 (segment (start 133.096 72.898) (end 133.096 69.694704) (width 0.25) (layer "B.Cu") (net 16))
 (segment (start 132.235296 68.834) (end 130.302 68.834) (width 0.25) (layer "B.Cu") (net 16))
 (segment (start 127.254 73.914) (end 132.08 73.914) (width 0.25) (layer "B.Cu") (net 16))
 (segment (start 132.08 73.914) (end 133.096 72.898) (width 0.25) (layer "B.Cu") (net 16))
 (segment (start 121.92 79.248) (end 127.254 73.914) (width 0.25) (layer "B.Cu") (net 16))
 (segment (start 130.302 68.834) (end 129.032 70.104) (width 0.25) (layer "B.Cu") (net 16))
 (segment (start 133.096 69.694704) (end 132.235296 68.834) (width 0.25) (layer "B.Cu") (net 16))
 (segment (start 121.92 84.8275) (end 121.92 79.248) (width 0.25) (layer "B.Cu") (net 16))
 (segment (start 121.86152 89.96598) (end 120.116 91.7115) (width 0.25) (layer "F.Cu") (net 18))
 (segment (start 130.536289 81.299711) (end 124.568007 81.299711) (width 0.25) (layer "F.Cu") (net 18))
 (segment (start 121.86152 84.006198) (end 121.86152 89.96598) (width 0.25) (layer "F.Cu") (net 18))
 (segment (start 131.572 80.264) (end 130.536289 81.299711) (width 0.25) (layer "F.Cu") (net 18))
 (segment (start 124.568007 81.299711) (end 121.86152 84.006198) (width 0.25) (layer "F.Cu") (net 18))
 (segment (start 145.542 86.614) (end 145.542 80.772) (width 0.25) (layer "B.Cu") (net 20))
 (segment (start 139.192 92.964) (end 145.542 86.614) (width 0.25) (layer "B.Cu") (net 20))
 (segment (start 120.116 96.7915) (end 123.9435 92.964) (width 0.25) (layer "B.Cu") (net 20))
 (segment (start 123.9435 92.964) (end 139.192 92.964) (width 0.25) (layer "B.Cu") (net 20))
 (segment (start 149.86 76.454) (end 153.162 76.454) (width 0.25) (layer "B.Cu") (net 20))
 (segment (start 153.162 76.454) (end 154.432 75.184) (width 0.25) (layer "B.Cu") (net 20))
 (segment (start 145.542 80.772) (end 149.86 76.454) (width 0.25) (layer "B.Cu") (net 20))
 (segment (start 157.226 77.978) (end 157.226 86.36) (width 0.25) (layer "F.Cu") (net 21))
 (segment (start 157.226 86.36) (end 153.67 89.916) (width 0.25) (layer "F.Cu") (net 21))
 (segment (start 151.892 77.724) (end 153.162 76.454) (width 0.25) (layer "F.Cu") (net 21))
 (segment (start 140.1905 96.7915) (end 135.356 96.7915) (width 0.25) (layer "F.Cu") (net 21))
 (segment (start 153.67 89.916) (end 147.066 89.916) (width 0.25) (layer "F.Cu") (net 21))
 (segment (start 153.162 76.454) (end 155.702 76.454) (width 0.25) (layer "F.Cu") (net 21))
 (segment (start 155.702 76.454) (end 157.226 77.978) (width 0.25) (layer "F.Cu") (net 21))
 (segment (start 147.066 89.916) (end 140.1905 96.7915) (width 0.25) (layer "F.Cu") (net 21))
 (segment (start 156.32696 85.987604) (end 156.32696 80.694242) (width 0.25) (layer "F.Cu") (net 23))
 (segment (start 156.32696 80.694242) (end 154.861007 79.228289) (width 0.25) (layer "F.Cu") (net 23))
 (segment (start 154.861007 79.228289) (end 152.927711 79.228289) (width 0.25) (layer "F.Cu") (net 23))
 (segment (start 153.297604 89.01696) (end 156.32696 85.987604) (width 0.25) (layer "F.Cu") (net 23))
 (segment (start 135.356 91.7115) (end 143.999064 91.7115) (width 0.25) (layer "F.Cu") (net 23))
 (segment (start 143.999064 91.7115) (end 146.693606 89.01696) (width 0.25) (layer "F.Cu") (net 23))
 (segment (start 146.693606 89.01696) (end 153.297604 89.01696) (width 0.25) (layer "F.Cu") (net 23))
 (segment (start 152.927711 79.228289) (end 151.892 80.264) (width 0.25) (layer "F.Cu") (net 23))
 (segment (start 129.032 85.09) (end 130.5735 86.6315) (width 0.25) (layer "F.Cu") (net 25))
 (segment (start 129.032 82.804) (end 129.032 85.09) (width 0.25) (layer "F.Cu") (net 25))
 (segment (start 130.5735 86.6315) (end 135.356 86.6315) (width 0.25) (layer "F.Cu") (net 25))
 (segment (start 149.86 84.074) (end 150.856289 83.077711) (width 0.25) (layer "F.Cu") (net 27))
 (segment (start 137.1775 81.5515) (end 137.922 82.296) (width 0.25) (layer "F.Cu") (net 27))
 (segment (start 137.922 82.296) (end 137.922 83.312) (width 0.25) (layer "F.Cu") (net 27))
 (segment (start 150.856289 83.077711) (end 150.856289 82.335422) (width 0.25) (layer "F.Cu") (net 27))
 (segment (start 151.423422 81.768289) (end 153.396289 81.768289) (width 0.25) (layer "F.Cu") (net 27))
 (segment (start 150.856289 82.335422) (end 151.423422 81.768289) (width 0.25) (layer "F.Cu") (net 27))
 (segment (start 135.356 81.5515) (end 137.1775 81.5515) (width 0.25) (layer "F.Cu") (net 27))
 (segment (start 153.396289 81.768289) (end 154.432 82.804) (width 0.25) (layer "F.Cu") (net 27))
 (segment (start 137.922 83.312) (end 138.684 84.074) (width 0.25) (layer "F.Cu") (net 27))
 (segment (start 138.684 84.074) (end 149.86 84.074) (width 0.25) (layer "F.Cu") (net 27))
 (segment (start 139.1835 72.644) (end 135.356 76.4715) (width 0.25) (layer "F.Cu") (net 29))
 (segment (start 151.892 72.644) (end 139.1835 72.644) (width 0.25) (layer "F.Cu") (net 29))
 (segment (start 151.892 70.104) (end 136.6435 70.104) (width 0.25) (layer "F.Cu") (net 31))
 (segment (start 136.6435 70.104) (end 135.356 71.3915) (width 0.25) (layer "F.Cu") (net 31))
 (segment (start 136.6085 67.564) (end 135.356 66.3115) (width 0.25) (layer "F.Cu") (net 33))
 (segment (start 151.892 67.564) (end 136.6085 67.564) (width 0.25) (layer "F.Cu") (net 33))
 (segment (start 137.922 61.722) (end 137.4315 61.2315) (width 0.25) (layer "F.Cu") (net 35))
 (segment (start 137.922 64.008) (end 137.922 61.722) (width 0.25) (layer "F.Cu") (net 35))
 (segment (start 138.938 65.024) (end 137.922 64.008) (width 0.25) (layer "F.Cu") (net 35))
 (segment (start 137.4315 61.2315) (end 135.356 61.2315) (width 0.25) (layer "F.Cu") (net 35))
 (segment (start 151.892 65.024) (end 138.938 65.024) (width 0.25) (layer "F.Cu") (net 35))
 (segment (start 133.3675 58.6915) (end 132.842 59.217) (width 0.25) (layer "F.Cu") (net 36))
 (segment (start 132.842 78.74) (end 134.366 80.264) (width 0.25) (layer "F.Cu") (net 36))
 (segment (start 134.366 80.264) (end 137.668 80.264) (width 0.25) (layer "F.Cu") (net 36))
 (segment (start 137.668 80.264) (end 139.192 81.788) (width 0.25) (layer "F.Cu") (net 36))
 (segment (start 135.356 58.6915) (end 133.3675 58.6915) (width 0.25) (layer "F.Cu") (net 36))
 (segment (start 132.842 59.217) (end 132.842 78.74) (width 0.25) (layer "F.Cu") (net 36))
 (segment (start 139.192 81.788) (end 139.192 82.804) (width 0.25) (layer "F.Cu") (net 36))
 (segment (start 140.687789 73.679711) (end 135.356 79.0115) (width 0.25) (layer "F.Cu") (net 28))
 (segment (start 153.396289 73.679711) (end 140.687789 73.679711) (width 0.25) (layer "F.Cu") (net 28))
 (segment (start 154.432 72.644) (end 153.396289 73.679711) (width 0.25) (layer "F.Cu") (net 28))
 (segment (start 154.432 70.104) (end 153.396289 71.139711) (width 0.25) (layer "F.Cu") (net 30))
 (segment (start 153.396289 71.139711) (end 138.147789 71.139711) (width 0.25) (layer "F.Cu") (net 30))
 (segment (start 138.147789 71.139711) (end 135.356 73.9315) (width 0.25) (layer "F.Cu") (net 30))
 (segment (start 153.1445 68.8515) (end 135.356 68.8515) (width 0.25) (layer "F.Cu") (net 32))
 (segment (start 154.432 67.564) (end 153.1445 68.8515) (width 0.25) (layer "F.Cu") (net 32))
 (segment (start 154.432 65.024) (end 153.396289 66.059711) (width 0.25) (layer "F.Cu") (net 34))
 (segment (start 153.396289 66.059711) (end 137.644211 66.059711) (width 0.25) (layer "F.Cu") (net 34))
 (segment (start 137.644211 66.059711) (end 135.356 63.7715) (width 0.25) (layer "F.Cu") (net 34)))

